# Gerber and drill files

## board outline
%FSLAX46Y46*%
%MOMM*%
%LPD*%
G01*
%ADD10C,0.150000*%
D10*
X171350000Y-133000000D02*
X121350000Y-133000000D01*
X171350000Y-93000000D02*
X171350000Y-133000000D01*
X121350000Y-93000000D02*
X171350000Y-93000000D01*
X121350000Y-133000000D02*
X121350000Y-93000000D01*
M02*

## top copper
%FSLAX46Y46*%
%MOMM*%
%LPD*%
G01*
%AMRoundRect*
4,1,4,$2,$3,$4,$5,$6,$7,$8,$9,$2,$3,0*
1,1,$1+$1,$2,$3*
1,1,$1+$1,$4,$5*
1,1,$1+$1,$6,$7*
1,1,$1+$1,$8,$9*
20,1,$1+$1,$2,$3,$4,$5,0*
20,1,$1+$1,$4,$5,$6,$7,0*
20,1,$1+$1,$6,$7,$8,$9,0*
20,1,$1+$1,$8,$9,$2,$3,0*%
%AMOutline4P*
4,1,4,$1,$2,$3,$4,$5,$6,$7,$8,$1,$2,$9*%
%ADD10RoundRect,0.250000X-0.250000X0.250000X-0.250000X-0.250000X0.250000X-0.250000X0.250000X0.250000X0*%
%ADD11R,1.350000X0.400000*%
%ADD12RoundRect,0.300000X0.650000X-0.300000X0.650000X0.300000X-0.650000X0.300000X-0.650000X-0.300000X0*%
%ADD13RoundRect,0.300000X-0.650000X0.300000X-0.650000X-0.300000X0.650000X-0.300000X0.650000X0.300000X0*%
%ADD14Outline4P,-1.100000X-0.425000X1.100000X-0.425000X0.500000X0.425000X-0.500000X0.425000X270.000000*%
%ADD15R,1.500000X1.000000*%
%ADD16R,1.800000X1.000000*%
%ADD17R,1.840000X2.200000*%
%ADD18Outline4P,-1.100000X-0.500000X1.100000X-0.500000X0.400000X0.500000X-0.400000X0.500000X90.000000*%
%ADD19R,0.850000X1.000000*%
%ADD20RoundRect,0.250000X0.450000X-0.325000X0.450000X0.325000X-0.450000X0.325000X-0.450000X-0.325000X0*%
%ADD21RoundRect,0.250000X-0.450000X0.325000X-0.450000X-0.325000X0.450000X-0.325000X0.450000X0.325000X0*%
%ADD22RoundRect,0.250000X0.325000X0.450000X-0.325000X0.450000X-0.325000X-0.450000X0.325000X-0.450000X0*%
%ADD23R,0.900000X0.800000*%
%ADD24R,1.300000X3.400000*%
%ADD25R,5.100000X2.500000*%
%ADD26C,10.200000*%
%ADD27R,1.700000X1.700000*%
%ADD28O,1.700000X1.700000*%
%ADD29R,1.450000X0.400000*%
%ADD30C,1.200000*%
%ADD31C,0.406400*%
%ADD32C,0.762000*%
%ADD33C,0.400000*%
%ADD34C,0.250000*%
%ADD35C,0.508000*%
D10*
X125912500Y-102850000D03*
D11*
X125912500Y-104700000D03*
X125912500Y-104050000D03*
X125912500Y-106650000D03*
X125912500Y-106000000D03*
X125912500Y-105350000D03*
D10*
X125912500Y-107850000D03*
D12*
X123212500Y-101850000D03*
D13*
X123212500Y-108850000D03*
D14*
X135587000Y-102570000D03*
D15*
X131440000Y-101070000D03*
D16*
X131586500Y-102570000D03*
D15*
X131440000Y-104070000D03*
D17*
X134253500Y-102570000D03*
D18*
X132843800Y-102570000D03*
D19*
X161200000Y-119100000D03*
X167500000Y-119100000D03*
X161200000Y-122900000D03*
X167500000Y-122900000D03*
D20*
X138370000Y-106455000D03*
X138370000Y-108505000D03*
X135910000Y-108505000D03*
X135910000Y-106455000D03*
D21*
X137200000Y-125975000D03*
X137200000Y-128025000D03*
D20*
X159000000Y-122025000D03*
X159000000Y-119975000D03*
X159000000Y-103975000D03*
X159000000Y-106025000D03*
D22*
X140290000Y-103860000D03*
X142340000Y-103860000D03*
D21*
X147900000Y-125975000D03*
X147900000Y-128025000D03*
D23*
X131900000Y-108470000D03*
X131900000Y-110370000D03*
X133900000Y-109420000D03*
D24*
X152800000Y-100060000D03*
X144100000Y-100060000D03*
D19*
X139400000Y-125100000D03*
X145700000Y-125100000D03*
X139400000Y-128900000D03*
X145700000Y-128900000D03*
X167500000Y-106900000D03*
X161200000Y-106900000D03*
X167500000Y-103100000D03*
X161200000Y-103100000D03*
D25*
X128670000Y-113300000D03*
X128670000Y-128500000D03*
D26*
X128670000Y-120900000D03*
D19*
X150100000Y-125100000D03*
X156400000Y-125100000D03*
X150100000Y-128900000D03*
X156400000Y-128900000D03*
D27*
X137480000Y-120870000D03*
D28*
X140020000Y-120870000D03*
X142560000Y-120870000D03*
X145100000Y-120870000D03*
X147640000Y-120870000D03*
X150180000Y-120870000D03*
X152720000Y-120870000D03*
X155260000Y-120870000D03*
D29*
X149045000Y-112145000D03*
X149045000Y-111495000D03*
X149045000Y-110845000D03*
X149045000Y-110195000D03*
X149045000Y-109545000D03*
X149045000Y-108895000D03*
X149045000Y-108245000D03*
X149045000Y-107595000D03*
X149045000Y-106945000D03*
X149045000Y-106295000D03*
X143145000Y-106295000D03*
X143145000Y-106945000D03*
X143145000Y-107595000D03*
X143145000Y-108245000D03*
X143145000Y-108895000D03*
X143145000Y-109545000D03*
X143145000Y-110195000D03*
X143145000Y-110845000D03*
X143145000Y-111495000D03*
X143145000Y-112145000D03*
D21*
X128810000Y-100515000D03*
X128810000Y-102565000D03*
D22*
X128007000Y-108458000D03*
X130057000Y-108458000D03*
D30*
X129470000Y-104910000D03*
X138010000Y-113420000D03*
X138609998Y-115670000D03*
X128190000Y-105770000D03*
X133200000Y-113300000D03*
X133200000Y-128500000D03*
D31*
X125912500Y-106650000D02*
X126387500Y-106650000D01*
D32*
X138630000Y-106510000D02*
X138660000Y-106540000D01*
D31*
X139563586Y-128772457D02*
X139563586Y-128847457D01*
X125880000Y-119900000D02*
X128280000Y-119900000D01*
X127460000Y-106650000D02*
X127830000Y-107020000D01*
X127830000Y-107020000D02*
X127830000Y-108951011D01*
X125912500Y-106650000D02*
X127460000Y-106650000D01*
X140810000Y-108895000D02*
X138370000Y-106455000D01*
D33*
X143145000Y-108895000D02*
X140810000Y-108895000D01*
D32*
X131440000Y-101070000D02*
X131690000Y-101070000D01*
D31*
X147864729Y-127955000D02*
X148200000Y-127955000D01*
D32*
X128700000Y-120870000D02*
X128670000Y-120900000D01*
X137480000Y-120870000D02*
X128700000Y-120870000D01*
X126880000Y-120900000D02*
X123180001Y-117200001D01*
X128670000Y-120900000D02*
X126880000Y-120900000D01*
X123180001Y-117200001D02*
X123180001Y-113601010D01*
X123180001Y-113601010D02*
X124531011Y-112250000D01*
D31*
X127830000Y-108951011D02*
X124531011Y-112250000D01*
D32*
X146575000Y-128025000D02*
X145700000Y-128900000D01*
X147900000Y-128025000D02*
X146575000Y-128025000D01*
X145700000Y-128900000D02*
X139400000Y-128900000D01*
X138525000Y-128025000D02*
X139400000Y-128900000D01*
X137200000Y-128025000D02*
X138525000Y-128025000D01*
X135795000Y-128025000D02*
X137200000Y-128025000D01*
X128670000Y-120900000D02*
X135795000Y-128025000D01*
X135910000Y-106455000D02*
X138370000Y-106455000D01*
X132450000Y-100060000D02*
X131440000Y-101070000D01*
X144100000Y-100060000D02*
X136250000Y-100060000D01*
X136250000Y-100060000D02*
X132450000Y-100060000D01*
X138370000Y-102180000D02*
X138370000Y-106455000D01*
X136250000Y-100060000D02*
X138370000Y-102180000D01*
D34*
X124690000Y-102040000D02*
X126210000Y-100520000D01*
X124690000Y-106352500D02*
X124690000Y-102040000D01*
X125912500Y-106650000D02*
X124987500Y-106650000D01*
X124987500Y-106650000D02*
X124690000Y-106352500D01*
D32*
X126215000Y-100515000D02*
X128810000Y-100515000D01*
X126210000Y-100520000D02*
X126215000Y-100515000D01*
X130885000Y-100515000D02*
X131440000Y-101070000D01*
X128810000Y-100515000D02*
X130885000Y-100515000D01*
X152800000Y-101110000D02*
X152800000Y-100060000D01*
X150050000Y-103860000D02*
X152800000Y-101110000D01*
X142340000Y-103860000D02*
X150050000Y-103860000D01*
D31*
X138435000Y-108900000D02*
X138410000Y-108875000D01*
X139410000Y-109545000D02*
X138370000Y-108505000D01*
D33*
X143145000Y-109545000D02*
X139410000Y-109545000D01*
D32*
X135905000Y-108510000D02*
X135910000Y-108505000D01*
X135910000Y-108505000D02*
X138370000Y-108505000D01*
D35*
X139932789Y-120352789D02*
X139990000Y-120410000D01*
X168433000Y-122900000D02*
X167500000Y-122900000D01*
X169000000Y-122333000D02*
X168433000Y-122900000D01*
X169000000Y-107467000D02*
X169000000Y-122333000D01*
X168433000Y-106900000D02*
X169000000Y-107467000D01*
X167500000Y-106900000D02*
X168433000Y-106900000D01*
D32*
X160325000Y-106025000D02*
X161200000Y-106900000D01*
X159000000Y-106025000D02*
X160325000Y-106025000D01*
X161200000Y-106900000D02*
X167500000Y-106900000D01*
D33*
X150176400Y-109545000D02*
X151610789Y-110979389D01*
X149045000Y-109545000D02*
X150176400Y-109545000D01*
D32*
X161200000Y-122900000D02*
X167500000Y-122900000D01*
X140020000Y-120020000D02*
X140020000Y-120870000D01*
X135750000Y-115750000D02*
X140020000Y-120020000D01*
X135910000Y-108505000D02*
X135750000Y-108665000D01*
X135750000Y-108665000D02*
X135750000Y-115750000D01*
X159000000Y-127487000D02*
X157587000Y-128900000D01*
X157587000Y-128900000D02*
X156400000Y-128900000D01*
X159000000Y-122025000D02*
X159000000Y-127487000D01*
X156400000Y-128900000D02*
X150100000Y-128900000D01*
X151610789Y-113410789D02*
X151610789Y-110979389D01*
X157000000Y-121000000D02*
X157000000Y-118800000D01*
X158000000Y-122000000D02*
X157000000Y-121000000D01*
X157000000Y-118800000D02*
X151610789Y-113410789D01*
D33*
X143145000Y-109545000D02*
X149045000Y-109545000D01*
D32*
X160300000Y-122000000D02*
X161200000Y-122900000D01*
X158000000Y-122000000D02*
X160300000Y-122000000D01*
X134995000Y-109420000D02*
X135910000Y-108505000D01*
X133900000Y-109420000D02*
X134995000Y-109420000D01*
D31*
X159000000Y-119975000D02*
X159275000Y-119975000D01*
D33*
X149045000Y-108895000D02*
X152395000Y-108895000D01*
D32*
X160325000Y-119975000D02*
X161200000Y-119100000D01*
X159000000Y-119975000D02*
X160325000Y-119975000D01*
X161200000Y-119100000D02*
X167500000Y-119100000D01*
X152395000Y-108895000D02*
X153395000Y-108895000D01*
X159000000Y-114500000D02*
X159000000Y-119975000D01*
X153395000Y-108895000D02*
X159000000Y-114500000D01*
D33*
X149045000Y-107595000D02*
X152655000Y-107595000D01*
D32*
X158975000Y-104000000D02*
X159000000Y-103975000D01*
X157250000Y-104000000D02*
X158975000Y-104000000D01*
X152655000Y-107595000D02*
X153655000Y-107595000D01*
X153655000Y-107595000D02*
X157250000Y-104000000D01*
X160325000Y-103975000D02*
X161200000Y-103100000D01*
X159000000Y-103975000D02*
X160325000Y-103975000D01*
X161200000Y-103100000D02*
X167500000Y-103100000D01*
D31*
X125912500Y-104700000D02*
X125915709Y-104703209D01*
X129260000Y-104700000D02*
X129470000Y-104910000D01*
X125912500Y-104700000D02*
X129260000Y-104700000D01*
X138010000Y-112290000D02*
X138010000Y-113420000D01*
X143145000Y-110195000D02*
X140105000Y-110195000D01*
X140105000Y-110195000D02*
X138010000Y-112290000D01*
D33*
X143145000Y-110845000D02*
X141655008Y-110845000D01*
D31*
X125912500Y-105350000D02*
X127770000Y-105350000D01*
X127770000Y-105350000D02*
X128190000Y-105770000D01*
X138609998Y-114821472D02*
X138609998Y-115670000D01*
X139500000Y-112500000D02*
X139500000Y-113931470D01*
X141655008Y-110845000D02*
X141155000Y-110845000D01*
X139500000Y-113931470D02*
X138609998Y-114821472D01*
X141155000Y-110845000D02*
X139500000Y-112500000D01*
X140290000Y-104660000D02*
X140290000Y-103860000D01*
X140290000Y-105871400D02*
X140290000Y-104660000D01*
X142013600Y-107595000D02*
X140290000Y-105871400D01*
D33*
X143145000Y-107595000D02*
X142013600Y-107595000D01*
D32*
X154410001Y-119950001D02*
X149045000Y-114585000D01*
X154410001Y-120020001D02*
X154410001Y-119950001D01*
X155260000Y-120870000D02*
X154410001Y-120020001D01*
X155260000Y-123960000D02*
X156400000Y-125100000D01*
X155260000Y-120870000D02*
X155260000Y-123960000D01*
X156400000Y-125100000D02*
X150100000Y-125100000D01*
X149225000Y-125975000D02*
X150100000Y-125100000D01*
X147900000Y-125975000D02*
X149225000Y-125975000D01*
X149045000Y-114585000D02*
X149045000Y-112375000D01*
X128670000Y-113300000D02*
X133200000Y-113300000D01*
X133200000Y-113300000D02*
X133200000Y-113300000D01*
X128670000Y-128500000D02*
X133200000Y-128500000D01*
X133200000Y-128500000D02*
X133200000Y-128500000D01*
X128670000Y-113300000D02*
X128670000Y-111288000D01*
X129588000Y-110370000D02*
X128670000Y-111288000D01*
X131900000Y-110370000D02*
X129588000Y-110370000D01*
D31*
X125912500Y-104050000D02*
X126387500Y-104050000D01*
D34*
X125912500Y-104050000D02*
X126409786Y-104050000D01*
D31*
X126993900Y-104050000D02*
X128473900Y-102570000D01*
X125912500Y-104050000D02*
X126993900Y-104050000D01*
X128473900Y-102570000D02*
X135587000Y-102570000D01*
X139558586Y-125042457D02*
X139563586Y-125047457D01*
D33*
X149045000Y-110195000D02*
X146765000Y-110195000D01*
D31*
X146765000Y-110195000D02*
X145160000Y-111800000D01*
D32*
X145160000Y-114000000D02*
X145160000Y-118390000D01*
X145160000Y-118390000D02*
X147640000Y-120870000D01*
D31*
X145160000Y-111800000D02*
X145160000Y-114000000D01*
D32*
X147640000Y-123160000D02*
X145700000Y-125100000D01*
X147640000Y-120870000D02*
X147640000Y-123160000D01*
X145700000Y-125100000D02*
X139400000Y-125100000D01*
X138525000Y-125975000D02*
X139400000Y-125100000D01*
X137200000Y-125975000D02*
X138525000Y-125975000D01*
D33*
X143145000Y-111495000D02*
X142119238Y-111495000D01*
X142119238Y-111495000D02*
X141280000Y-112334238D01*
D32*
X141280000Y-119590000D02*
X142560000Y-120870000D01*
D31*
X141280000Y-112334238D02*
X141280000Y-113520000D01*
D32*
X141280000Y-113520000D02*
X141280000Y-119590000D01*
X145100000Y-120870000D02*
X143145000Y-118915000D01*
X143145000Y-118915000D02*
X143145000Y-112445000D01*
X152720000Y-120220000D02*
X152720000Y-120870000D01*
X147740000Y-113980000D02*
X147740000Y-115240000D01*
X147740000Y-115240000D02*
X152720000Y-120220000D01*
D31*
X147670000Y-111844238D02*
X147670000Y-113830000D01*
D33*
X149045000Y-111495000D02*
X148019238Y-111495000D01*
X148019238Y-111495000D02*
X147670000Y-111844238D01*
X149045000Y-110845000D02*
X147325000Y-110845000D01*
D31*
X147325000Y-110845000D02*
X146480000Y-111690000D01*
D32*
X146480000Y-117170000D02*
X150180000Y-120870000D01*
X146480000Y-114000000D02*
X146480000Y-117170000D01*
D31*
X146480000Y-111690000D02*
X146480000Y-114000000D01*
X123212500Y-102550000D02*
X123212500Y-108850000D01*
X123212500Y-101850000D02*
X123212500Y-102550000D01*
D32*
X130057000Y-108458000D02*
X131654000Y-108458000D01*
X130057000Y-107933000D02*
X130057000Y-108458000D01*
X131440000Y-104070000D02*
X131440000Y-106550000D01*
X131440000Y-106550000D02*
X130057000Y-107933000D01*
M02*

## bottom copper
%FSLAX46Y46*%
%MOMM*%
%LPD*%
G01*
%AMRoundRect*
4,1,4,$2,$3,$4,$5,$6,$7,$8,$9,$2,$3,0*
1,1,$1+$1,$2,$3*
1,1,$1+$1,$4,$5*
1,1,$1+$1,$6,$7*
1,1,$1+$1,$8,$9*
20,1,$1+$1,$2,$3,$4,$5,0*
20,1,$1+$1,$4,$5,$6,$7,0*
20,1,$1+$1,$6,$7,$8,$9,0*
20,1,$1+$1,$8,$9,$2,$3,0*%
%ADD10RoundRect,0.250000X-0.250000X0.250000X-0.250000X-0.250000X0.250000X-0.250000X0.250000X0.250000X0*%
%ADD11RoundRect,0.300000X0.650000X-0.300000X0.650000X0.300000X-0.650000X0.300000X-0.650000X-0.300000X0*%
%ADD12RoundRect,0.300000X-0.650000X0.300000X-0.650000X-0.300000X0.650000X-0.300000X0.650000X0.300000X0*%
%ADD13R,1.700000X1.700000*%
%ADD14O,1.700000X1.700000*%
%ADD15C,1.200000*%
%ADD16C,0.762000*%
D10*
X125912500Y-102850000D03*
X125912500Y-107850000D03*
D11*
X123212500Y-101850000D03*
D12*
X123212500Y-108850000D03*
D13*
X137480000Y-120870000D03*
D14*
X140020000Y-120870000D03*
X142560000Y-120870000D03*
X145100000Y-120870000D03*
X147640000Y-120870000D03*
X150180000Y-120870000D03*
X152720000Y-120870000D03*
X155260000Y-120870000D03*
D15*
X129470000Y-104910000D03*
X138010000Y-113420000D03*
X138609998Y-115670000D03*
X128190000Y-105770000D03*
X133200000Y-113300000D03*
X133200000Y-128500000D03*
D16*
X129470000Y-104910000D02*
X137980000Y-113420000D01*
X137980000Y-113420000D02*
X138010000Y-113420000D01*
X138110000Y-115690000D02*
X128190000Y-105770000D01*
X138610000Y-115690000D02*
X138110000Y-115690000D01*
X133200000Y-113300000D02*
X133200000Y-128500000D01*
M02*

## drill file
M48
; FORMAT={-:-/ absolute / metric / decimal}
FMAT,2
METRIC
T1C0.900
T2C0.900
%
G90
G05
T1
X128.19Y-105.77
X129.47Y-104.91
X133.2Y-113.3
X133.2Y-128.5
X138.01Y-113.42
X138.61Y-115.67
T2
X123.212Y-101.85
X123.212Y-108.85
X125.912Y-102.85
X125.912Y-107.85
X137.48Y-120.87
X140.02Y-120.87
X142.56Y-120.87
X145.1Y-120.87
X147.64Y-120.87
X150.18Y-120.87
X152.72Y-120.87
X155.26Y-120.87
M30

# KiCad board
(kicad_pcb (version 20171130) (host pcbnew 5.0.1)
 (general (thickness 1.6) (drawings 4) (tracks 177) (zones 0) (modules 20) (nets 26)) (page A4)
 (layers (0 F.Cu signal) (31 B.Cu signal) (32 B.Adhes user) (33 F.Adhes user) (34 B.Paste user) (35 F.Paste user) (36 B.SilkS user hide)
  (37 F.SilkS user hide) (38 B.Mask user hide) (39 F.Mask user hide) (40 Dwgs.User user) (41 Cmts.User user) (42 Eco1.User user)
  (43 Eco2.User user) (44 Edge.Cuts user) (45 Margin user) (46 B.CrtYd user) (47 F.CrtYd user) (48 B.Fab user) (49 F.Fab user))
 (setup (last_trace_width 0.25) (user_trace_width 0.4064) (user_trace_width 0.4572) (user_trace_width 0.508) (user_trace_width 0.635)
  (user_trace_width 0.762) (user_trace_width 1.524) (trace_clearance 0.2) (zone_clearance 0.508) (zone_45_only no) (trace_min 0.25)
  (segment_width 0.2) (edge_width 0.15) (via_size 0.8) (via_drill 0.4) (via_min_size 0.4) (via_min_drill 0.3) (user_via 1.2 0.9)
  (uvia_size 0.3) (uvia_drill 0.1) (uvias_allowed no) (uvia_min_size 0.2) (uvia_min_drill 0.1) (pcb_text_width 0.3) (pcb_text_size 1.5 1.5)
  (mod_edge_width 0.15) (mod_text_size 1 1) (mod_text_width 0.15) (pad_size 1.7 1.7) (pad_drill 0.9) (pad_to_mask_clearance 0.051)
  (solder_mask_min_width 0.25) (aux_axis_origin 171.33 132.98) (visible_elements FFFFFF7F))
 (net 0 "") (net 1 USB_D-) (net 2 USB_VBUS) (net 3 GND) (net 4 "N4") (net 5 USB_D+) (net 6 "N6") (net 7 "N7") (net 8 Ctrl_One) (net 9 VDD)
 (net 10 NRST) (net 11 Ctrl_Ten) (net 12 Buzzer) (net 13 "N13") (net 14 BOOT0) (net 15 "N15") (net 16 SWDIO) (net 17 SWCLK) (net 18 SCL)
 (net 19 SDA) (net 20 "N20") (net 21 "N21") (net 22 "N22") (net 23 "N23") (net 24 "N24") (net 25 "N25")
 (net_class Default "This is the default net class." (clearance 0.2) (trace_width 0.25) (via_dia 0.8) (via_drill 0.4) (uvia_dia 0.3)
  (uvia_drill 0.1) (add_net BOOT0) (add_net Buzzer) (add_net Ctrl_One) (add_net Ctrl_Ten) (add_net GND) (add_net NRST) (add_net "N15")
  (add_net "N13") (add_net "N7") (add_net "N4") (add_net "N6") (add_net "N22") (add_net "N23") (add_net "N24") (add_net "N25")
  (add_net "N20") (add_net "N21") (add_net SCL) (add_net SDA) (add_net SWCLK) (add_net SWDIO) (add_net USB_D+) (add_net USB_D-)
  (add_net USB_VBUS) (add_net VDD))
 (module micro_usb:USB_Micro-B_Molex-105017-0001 (layer F.Cu) (at 124.45 105.35 270)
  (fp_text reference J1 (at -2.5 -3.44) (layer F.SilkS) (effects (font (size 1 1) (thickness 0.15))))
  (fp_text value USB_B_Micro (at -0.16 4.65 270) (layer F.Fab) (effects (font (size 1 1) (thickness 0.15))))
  (pad "" thru_hole roundrect (at -2.5 -1.4625 270) (size 1 1) (drill 0.9) (layers *.Cu *.Mask) (roundrect_rratio 0.25))
  (pad 2 smd rect (at -0.65 -1.4625 270) (size 0.4 1.35) (layers F.Cu F.Paste F.Mask) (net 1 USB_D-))
  (pad 1 smd rect (at -1.3 -1.4625 270) (size 0.4 1.35) (layers F.Cu F.Paste F.Mask) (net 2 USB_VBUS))
  (pad 5 smd rect (at 1.3 -1.4625 270) (size 0.4 1.35) (layers F.Cu F.Paste F.Mask) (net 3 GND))
  (pad 4 smd rect (at 0.65 -1.4625 270) (size 0.4 1.35) (layers F.Cu F.Paste F.Mask) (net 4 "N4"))
  (pad 3 smd rect (at 0 -1.4625 270) (size 0.4 1.35) (layers F.Cu F.Paste F.Mask) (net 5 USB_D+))
  (pad "" thru_hole roundrect (at 2.5 -1.4625 270) (size 1 1) (drill 0.9) (layers *.Cu *.Mask) (roundrect_rratio 0.25))
  (pad 6 thru_hole roundrect (at -3.5 1.2375 90) (size 1.2 1.9) (drill 0.9) (layers *.Cu *.Mask) (roundrect_rratio 0.25) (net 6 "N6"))
  (pad 6 thru_hole roundrect (at 3.5 1.2375 270) (size 1.2 1.9) (drill 0.9) (layers *.Cu *.Mask) (roundrect_rratio 0.25) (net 6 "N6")))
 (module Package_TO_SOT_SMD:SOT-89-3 (layer F.Cu) (at 132.92 102.57)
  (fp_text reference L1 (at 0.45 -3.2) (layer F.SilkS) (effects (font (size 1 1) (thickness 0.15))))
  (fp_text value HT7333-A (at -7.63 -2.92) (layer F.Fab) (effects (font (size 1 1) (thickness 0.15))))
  (pad 2 smd trapezoid (at 2.667 0 270) (size 1.6 0.85) (rect_delta 0 0.6) (layers F.Cu F.Paste F.Mask) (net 2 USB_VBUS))
  (pad 1 smd rect (at -1.48 -1.5 270) (size 1 1.5) (layers F.Cu F.Paste F.Mask) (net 3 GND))
  (pad 2 smd rect (at -1.3335 0 270) (size 1 1.8) (layers F.Cu F.Paste F.Mask) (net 2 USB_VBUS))
  (pad 3 smd rect (at -1.48 1.5 270) (size 1 1.5) (layers F.Cu F.Paste F.Mask) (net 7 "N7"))
  (pad 2 smd rect (at 1.3335 0 270) (size 2.2 1.84) (layers F.Cu F.Paste F.Mask) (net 2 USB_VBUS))
  (pad 2 smd trapezoid (at -0.0762 0 90) (size 1.5 1) (rect_delta 0 0.7) (layers F.Cu F.Paste F.Mask) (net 2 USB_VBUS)))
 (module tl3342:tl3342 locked (layer F.Cu) (at 164.35 121)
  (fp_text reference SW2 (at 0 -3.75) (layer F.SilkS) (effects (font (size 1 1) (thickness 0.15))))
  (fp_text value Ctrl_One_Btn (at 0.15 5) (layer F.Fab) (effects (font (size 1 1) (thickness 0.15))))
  (pad 1 smd rect (at -3.15 -1.9) (size 0.85 1) (layers F.Cu F.Paste F.Mask) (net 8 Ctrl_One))
  (pad 1 smd rect (at 3.15 -1.9) (size 0.85 1) (layers F.Cu F.Paste F.Mask) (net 8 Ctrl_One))
  (pad 2 smd rect (at -3.15 1.9) (size 0.85 1) (layers F.Cu F.Paste F.Mask) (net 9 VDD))
  (pad 2 smd rect (at 3.15 1.9) (size 0.85 1) (layers F.Cu F.Paste F.Mask) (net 9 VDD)))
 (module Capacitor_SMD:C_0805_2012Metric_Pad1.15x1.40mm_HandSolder (layer F.Cu) (at 138.37 107.48 90)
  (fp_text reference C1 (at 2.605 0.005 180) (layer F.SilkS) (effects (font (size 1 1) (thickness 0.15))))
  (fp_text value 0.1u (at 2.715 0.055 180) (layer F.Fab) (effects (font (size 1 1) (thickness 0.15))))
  (pad 2 smd roundrect (at 1.025 0 90) (size 1.15 1.4) (layers F.Cu F.Paste F.Mask) (roundrect_rratio 0.217391) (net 3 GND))
  (pad 1 smd roundrect (at -1.025 0 90) (size 1.15 1.4) (layers F.Cu F.Paste F.Mask) (roundrect_rratio 0.217391) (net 9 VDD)))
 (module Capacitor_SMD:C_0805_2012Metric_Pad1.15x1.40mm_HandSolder (layer F.Cu) (at 135.91 107.48 90)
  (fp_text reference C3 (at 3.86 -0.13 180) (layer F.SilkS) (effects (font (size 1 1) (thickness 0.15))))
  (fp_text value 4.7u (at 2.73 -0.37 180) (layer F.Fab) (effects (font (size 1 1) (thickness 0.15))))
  (pad 1 smd roundrect (at -1.025 0 90) (size 1.15 1.4) (layers F.Cu F.Paste F.Mask) (roundrect_rratio 0.217391) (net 9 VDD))
  (pad 2 smd roundrect (at 1.025 0 90) (size 1.15 1.4) (layers F.Cu F.Paste F.Mask) (roundrect_rratio 0.217391) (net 3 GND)))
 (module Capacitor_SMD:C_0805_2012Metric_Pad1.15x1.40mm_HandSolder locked (layer F.Cu) (at 137.2 127 270)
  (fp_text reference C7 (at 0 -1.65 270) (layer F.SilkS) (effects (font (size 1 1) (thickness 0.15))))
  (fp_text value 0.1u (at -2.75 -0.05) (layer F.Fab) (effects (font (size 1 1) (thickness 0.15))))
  (pad 1 smd roundrect (at -1.025 0 270) (size 1.15 1.4) (layers F.Cu F.Paste F.Mask) (roundrect_rratio 0.217391) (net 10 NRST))
  (pad 2 smd roundrect (at 1.025 0 270) (size 1.15 1.4) (layers F.Cu F.Paste F.Mask) (roundrect_rratio 0.217391) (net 3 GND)))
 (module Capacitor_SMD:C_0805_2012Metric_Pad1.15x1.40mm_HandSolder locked (layer F.Cu) (at 159 121 90)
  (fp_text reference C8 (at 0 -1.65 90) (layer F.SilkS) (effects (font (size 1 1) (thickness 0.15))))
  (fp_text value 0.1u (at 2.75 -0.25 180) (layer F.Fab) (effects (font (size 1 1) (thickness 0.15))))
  (pad 1 smd roundrect (at -1.025 0 90) (size 1.15 1.4) (layers F.Cu F.Paste F.Mask) (roundrect_rratio 0.217391) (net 9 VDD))
  (pad 2 smd roundrect (at 1.025 0 90) (size 1.15 1.4) (layers F.Cu F.Paste F.Mask) (roundrect_rratio 0.217391) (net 8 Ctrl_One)))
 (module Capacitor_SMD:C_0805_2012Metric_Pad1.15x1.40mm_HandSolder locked (layer F.Cu) (at 159 105 90)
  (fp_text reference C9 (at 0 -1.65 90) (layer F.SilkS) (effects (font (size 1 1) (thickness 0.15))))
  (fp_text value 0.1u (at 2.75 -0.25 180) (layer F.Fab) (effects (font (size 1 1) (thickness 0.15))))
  (pad 2 smd roundrect (at 1.025 0 90) (size 1.15 1.4) (layers F.Cu F.Paste F.Mask) (roundrect_rratio 0.217391) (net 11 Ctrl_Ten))
  (pad 1 smd roundrect (at -1.025 0 90) (size 1.15 1.4) (layers F.Cu F.Paste F.Mask) (roundrect_rratio 0.217391) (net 9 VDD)))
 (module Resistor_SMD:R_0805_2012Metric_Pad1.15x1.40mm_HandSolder (layer F.Cu) (at 141.315 103.86 180)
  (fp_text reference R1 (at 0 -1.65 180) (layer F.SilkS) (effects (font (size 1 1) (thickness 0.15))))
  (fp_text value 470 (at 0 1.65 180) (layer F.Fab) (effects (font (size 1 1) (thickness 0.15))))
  (pad 2 smd roundrect (at 1.025 0 180) (size 1.15 1.4) (layers F.Cu F.Paste F.Mask) (roundrect_rratio 0.217391) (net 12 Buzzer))
  (pad 1 smd roundrect (at -1.025 0 180) (size 1.15 1.4) (layers F.Cu F.Paste F.Mask) (roundrect_rratio 0.217391) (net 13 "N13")))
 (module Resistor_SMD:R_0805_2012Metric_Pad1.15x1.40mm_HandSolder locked (layer F.Cu) (at 147.9 127 270)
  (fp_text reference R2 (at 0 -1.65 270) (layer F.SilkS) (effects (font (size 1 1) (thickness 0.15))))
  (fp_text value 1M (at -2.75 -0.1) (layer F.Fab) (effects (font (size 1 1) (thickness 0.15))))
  (pad 1 smd roundrect (at -1.025 0 270) (size 1.15 1.4) (layers F.Cu F.Paste F.Mask) (roundrect_rratio 0.217391) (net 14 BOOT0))
  (pad 2 smd roundrect (at 1.025 0 270) (size 1.15 1.4) (layers F.Cu F.Paste F.Mask) (roundrect_rratio 0.217391) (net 3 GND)))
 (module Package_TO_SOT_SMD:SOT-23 (layer F.Cu) (at 132.9 109.42)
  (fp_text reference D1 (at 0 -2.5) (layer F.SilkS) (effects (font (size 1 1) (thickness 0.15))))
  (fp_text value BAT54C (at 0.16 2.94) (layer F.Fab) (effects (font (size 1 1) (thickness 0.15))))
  (pad 1 smd rect (at -1 -0.95) (size 0.9 0.8) (layers F.Cu F.Paste F.Mask) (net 7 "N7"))
  (pad 2 smd rect (at -1 0.95) (size 0.9 0.8) (layers F.Cu F.Paste F.Mask) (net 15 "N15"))
  (pad 3 smd rect (at 1 0) (size 0.9 0.8) (layers F.Cu F.Paste F.Mask) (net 9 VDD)))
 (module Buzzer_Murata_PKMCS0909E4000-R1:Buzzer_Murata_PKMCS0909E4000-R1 (layer F.Cu) (at 148.45 100.06 180)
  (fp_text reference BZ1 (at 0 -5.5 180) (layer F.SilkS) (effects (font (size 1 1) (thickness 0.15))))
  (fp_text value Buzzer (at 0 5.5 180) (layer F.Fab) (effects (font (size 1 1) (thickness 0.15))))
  (pad 1 smd rect (at -4.35 0 180) (size 1.3 3.4) (layers F.Cu F.Paste F.Mask) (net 13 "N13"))
  (pad 2 smd rect (at 4.35 0 180) (size 1.3 3.4) (layers F.Cu F.Paste F.Mask) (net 3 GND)))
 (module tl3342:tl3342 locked (layer F.Cu) (at 142.55 127)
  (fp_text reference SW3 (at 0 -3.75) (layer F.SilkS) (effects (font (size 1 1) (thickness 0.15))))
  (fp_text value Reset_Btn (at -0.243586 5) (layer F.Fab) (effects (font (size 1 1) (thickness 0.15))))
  (pad 1 smd rect (at -3.15 -1.9) (size 0.85 1) (layers F.Cu F.Paste F.Mask) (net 10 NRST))
  (pad 1 smd rect (at 3.15 -1.9) (size 0.85 1) (layers F.Cu F.Paste F.Mask) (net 10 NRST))
  (pad 2 smd rect (at -3.15 1.9) (size 0.85 1) (layers F.Cu F.Paste F.Mask) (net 3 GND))
  (pad 2 smd rect (at 3.15 1.9) (size 0.85 1) (layers F.Cu F.Paste F.Mask) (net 3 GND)))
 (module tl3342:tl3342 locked (layer F.Cu) (at 164.35 105)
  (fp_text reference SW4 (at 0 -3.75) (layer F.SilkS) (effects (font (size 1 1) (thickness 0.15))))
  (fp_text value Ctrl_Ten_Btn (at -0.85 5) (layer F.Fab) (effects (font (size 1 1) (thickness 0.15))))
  (pad 2 smd rect (at 3.15 1.9) (size 0.85 1) (layers F.Cu F.Paste F.Mask) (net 9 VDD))
  (pad 2 smd rect (at -3.15 1.9) (size 0.85 1) (layers F.Cu F.Paste F.Mask) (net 9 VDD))
  (pad 1 smd rect (at 3.15 -1.9) (size 0.85 1) (layers F.Cu F.Paste F.Mask) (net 11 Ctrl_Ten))
  (pad 1 smd rect (at -3.15 -1.9) (size 0.85 1) (layers F.Cu F.Paste F.Mask) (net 11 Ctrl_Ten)))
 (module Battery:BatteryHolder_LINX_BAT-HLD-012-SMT (layer F.Cu) (at 128.67 120.9 270)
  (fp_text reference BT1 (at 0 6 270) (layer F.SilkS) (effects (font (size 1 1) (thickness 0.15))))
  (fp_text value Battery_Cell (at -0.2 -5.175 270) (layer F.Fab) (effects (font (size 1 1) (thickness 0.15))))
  (pad 1 smd rect (at -7.6 0 270) (size 2.5 5.1) (layers F.Cu F.Paste F.Mask) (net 15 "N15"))
  (pad 1 smd rect (at 7.6 0 270) (size 2.5 5.1) (layers F.Cu F.Paste F.Mask) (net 15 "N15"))
  (pad 2 smd circle (at 0 0 270) (size 10.2 10.2) (layers F.Cu F.Paste F.Mask) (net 3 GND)))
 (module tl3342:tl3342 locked (layer F.Cu) (at 153.25 127)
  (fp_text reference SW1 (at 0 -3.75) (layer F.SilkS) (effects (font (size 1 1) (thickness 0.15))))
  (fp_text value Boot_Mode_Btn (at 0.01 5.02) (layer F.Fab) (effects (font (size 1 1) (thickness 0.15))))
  (pad 1 smd rect (at -3.15 -1.9) (size 0.85 1) (layers F.Cu F.Paste F.Mask) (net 14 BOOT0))
  (pad 1 smd rect (at 3.15 -1.9) (size 0.85 1) (layers F.Cu F.Paste F.Mask) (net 14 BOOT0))
  (pad 2 smd rect (at -3.15 1.9) (size 0.85 1) (layers F.Cu F.Paste F.Mask) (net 9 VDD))
  (pad 2 smd rect (at 3.15 1.9) (size 0.85 1) (layers F.Cu F.Paste F.Mask) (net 9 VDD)))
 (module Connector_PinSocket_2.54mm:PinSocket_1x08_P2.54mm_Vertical (layer F.Cu) (at 137.48 120.87 90)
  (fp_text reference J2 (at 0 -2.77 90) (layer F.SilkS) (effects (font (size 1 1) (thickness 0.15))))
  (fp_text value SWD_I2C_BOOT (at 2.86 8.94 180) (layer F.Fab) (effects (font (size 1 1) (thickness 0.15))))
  (pad 1 thru_hole rect (at 0 0 90) (size 1.7 1.7) (drill 0.9) (layers *.Cu *.Mask) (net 3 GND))
  (pad 2 thru_hole oval (at 0 2.54 90) (size 1.7 1.7) (drill 0.9) (layers *.Cu *.Mask) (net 9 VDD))
  (pad 3 thru_hole oval (at 0 5.08 90) (size 1.7 1.7) (drill 0.9) (layers *.Cu *.Mask) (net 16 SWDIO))
  (pad 4 thru_hole oval (at 0 7.62 90) (size 1.7 1.7) (drill 0.9) (layers *.Cu *.Mask) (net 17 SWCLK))
  (pad 5 thru_hole oval (at 0 10.16 90) (size 1.7 1.7) (drill 0.9) (layers *.Cu *.Mask) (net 10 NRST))
  (pad 6 thru_hole oval (at 0 12.7 90) (size 1.7 1.7) (drill 0.9) (layers *.Cu *.Mask) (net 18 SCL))
  (pad 7 thru_hole oval (at 0 15.24 90) (size 1.7 1.7) (drill 0.9) (layers *.Cu *.Mask) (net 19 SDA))
  (pad 8 thru_hole oval (at 0 17.78 90) (size 1.7 1.7) (drill 0.9) (layers *.Cu *.Mask) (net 14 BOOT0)))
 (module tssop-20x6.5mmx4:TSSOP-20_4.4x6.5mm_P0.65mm (layer F.Cu) (at 146.095 109.22 180)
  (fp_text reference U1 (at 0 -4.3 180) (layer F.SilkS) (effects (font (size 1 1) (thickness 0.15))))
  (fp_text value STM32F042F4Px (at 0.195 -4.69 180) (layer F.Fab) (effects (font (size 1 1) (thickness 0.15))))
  (pad 1 smd rect (at -2.95 -2.925 180) (size 1.45 0.4) (layers F.Cu F.Paste F.Mask) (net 14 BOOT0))
  (pad 2 smd rect (at -2.95 -2.275 180) (size 1.45 0.4) (layers F.Cu F.Paste F.Mask) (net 19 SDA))
  (pad 3 smd rect (at -2.95 -1.625 180) (size 1.45 0.4) (layers F.Cu F.Paste F.Mask) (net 18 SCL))
  (pad 4 smd rect (at -2.95 -0.975 180) (size 1.45 0.4) (layers F.Cu F.Paste F.Mask) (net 10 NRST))
  (pad 5 smd rect (at -2.95 -0.325 180) (size 1.45 0.4) (layers F.Cu F.Paste F.Mask) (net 9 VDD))
  (pad 6 smd rect (at -2.95 0.325 180) (size 1.45 0.4) (layers F.Cu F.Paste F.Mask) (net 8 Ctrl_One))
  (pad 7 smd rect (at -2.95 0.975 180) (size 1.45 0.4) (layers F.Cu F.Paste F.Mask) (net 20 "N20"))
  (pad 8 smd rect (at -2.95 1.625 180) (size 1.45 0.4) (layers F.Cu F.Paste F.Mask) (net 11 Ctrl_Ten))
  (pad 9 smd rect (at -2.95 2.275 180) (size 1.45 0.4) (layers F.Cu F.Paste F.Mask) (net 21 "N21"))
  (pad 10 smd rect (at -2.95 2.925 180) (size 1.45 0.4) (layers F.Cu F.Paste F.Mask) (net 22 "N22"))
  (pad 11 smd rect (at 2.95 2.925 180) (size 1.45 0.4) (layers F.Cu F.Paste F.Mask) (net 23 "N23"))
  (pad 12 smd rect (at 2.95 2.275 180) (size 1.45 0.4) (layers F.Cu F.Paste F.Mask) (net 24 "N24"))
  (pad 13 smd rect (at 2.95 1.625 180) (size 1.45 0.4) (layers F.Cu F.Paste F.Mask) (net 12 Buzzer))
  (pad 14 smd rect (at 2.95 0.975 180) (size 1.45 0.4) (layers F.Cu F.Paste F.Mask) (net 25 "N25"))
  (pad 15 smd rect (at 2.95 0.325 180) (size 1.45 0.4) (layers F.Cu F.Paste F.Mask) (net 3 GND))
  (pad 16 smd rect (at 2.95 -0.325 180) (size 1.45 0.4) (layers F.Cu F.Paste F.Mask) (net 9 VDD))
  (pad 17 smd rect (at 2.95 -0.975 180) (size 1.45 0.4) (layers F.Cu F.Paste F.Mask) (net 1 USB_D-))
  (pad 18 smd rect (at 2.95 -1.625 180) (size 1.45 0.4) (layers F.Cu F.Paste F.Mask) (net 5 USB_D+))
  (pad 19 smd rect (at 2.95 -2.275 180) (size 1.45 0.4) (layers F.Cu F.Paste F.Mask) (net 16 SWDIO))
  (pad 20 smd rect (at 2.95 -2.925 180) (size 1.45 0.4) (layers F.Cu F.Paste F.Mask) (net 17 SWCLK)))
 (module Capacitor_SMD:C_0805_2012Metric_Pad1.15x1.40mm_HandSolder (layer F.Cu) (at 128.81 101.54 270)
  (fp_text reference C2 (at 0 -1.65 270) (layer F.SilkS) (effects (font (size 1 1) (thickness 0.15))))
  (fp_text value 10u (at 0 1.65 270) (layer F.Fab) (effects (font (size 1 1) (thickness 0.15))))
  (pad 1 smd roundrect (at -1.025 0 270) (size 1.15 1.4) (layers F.Cu F.Paste F.Mask) (roundrect_rratio 0.217391) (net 3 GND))
  (pad 2 smd roundrect (at 1.025 0 270) (size 1.15 1.4) (layers F.Cu F.Paste F.Mask) (roundrect_rratio 0.217391) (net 2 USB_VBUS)))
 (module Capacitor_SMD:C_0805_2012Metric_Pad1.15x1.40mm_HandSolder (layer F.Cu) (at 129.032 108.458 180)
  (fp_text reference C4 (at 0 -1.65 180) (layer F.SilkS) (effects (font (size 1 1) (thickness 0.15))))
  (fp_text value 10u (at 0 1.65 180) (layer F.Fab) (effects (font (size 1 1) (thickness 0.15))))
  (pad 2 smd roundrect (at 1.025 0 180) (size 1.15 1.4) (layers F.Cu F.Paste F.Mask) (roundrect_rratio 0.217391) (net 3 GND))
  (pad 1 smd roundrect (at -1.025 0 180) (size 1.15 1.4) (layers F.Cu F.Paste F.Mask) (roundrect_rratio 0.217391) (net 7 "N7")))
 (gr_line (start 171.35 133) (end 121.35 133) (layer Edge.Cuts) (width 0.15))
 (gr_line (start 171.35 93) (end 171.35 133) (layer Edge.Cuts) (width 0.15))
 (gr_line (start 121.35 93) (end 171.35 93) (layer Edge.Cuts) (width 0.15))
 (gr_line (start 121.35 133) (end 121.35 93) (layer Edge.Cuts) (width 0.15))
 (segment (start 125.9125 106.65) (end 126.3875 106.65) (width 0.4064) (layer F.Cu) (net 3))
 (segment (start 138.63 106.51) (end 138.66 106.54) (width 0.762) (layer F.Cu) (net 3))
 (segment (start 139.563586 128.772457) (end 139.563586 128.847457) (width 0.4064) (layer F.Cu) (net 3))
 (segment (start 125.88 119.9) (end 128.28 119.9) (width 0.4064) (layer F.Cu) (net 3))
 (segment (start 127.46 106.65) (end 127.83 107.02) (width 0.4064) (layer F.Cu) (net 3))
 (segment (start 127.83 107.02) (end 127.83 108.951011) (width 0.4064) (layer F.Cu) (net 3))
 (segment (start 125.9125 106.65) (end 127.46 106.65) (width 0.4064) (layer F.Cu) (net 3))
 (segment (start 140.81 108.895) (end 138.37 106.455) (width 0.4064) (layer F.Cu) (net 3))
 (segment (start 143.145 108.895) (end 140.81 108.895) (width 0.4) (layer F.Cu) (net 3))
 (segment (start 131.44 101.07) (end 131.69 101.07) (width 0.762) (layer F.Cu) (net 3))
 (segment (start 147.864729 127.955) (end 148.2 127.955) (width 0.4064) (layer F.Cu) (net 3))
 (segment (start 128.7 120.87) (end 128.67 120.9) (width 0.762) (layer F.Cu) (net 3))
 (segment (start 137.48 120.87) (end 128.7 120.87) (width 0.762) (layer F.Cu) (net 3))
 (segment (start 126.88 120.9) (end 123.180001 117.200001) (width 0.762) (layer F.Cu) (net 3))
 (segment (start 128.67 120.9) (end 126.88 120.9) (width 0.762) (layer F.Cu) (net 3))
 (segment (start 123.180001 117.200001) (end 123.180001 113.60101) (width 0.762) (layer F.Cu) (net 3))
 (segment (start 123.180001 113.60101) (end 124.531011 112.25) (width 0.762) (layer F.Cu) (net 3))
 (segment (start 127.83 108.951011) (end 124.531011 112.25) (width 0.4064) (layer F.Cu) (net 3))
 (segment (start 146.575 128.025) (end 145.7 128.9) (width 0.762) (layer F.Cu) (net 3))
 (segment (start 147.9 128.025) (end 146.575 128.025) (width 0.762) (layer F.Cu) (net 3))
 (segment (start 145.7 128.9) (end 139.4 128.9) (width 0.762) (layer F.Cu) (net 3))
 (segment (start 138.525 128.025) (end 139.4 128.9) (width 0.762) (layer F.Cu) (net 3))
 (segment (start 137.2 128.025) (end 138.525 128.025) (width 0.762) (layer F.Cu) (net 3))
 (segment (start 135.795 128.025) (end 137.2 128.025) (width 0.762) (layer F.Cu) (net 3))
 (segment (start 128.67 120.9) (end 135.795 128.025) (width 0.762) (layer F.Cu) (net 3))
 (segment (start 135.91 106.455) (end 138.37 106.455) (width 0.762) (layer F.Cu) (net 3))
 (segment (start 132.45 100.06) (end 131.44 101.07) (width 0.762) (layer F.Cu) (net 3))
 (segment (start 144.1 100.06) (end 136.25 100.06) (width 0.762) (layer F.Cu) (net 3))
 (segment (start 136.25 100.06) (end 132.45 100.06) (width 0.762) (layer F.Cu) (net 3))
 (segment (start 138.37 102.18) (end 138.37 106.455) (width 0.762) (layer F.Cu) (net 3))
 (segment (start 136.25 100.06) (end 138.37 102.18) (width 0.762) (layer F.Cu) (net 3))
 (segment (start 124.69 102.04) (end 126.21 100.52) (width 0.25) (layer F.Cu) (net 3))
 (segment (start 124.69 106.3525) (end 124.69 102.04) (width 0.25) (layer F.Cu) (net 3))
 (segment (start 125.9125 106.65) (end 124.9875 106.65) (width 0.25) (layer F.Cu) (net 3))
 (segment (start 124.9875 106.65) (end 124.69 106.3525) (width 0.25) (layer F.Cu) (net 3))
 (segment (start 126.215 100.515) (end 128.81 100.515) (width 0.762) (layer F.Cu) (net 3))
 (segment (start 126.21 100.52) (end 126.215 100.515) (width 0.762) (layer F.Cu) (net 3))
 (segment (start 130.885 100.515) (end 131.44 101.07) (width 0.762) (layer F.Cu) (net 3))
 (segment (start 128.81 100.515) (end 130.885 100.515) (width 0.762) (layer F.Cu) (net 3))
 (segment (start 152.8 101.11) (end 152.8 100.06) (width 0.762) (layer F.Cu) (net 13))
 (segment (start 150.05 103.86) (end 152.8 101.11) (width 0.762) (layer F.Cu) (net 13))
 (segment (start 142.34 103.86) (end 150.05 103.86) (width 0.762) (layer F.Cu) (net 13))
 (segment (start 138.435 108.9) (end 138.41 108.875) (width 0.4064) (layer F.Cu) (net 9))
 (segment (start 139.41 109.545) (end 138.37 108.505) (width 0.4064) (layer F.Cu) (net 9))
 (segment (start 143.145 109.545) (end 139.41 109.545) (width 0.4) (layer F.Cu) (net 9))
 (segment (start 135.905 108.51) (end 135.91 108.505) (width 0.762) (layer F.Cu) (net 9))
 (segment (start 135.91 108.505) (end 138.37 108.505) (width 0.762) (layer F.Cu) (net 9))
 (segment (start 139.932789 120.352789) (end 139.99 120.41) (width 0.508) (layer F.Cu) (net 9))
 (segment (start 168.433 122.9) (end 167.5 122.9) (width 0.508) (layer F.Cu) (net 9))
 (segment (start 169 122.333) (end 168.433 122.9) (width 0.508) (layer F.Cu) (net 9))
 (segment (start 169 107.467) (end 169 122.333) (width 0.508) (layer F.Cu) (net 9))
 (segment (start 168.433 106.9) (end 169 107.467) (width 0.508) (layer F.Cu) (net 9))
 (segment (start 167.5 106.9) (end 168.433 106.9) (width 0.508) (layer F.Cu) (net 9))
 (segment (start 160.325 106.025) (end 161.2 106.9) (width 0.762) (layer F.Cu) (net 9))
 (segment (start 159 106.025) (end 160.325 106.025) (width 0.762) (layer F.Cu) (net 9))
 (segment (start 161.2 106.9) (end 167.5 106.9) (width 0.762) (layer F.Cu) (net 9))
 (segment (start 150.1764 109.545) (end 151.610789 110.979389) (width 0.4) (layer F.Cu) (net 9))
 (segment (start 149.045 109.545) (end 150.1764 109.545) (width 0.4) (layer F.Cu) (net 9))
 (segment (start 161.2 122.9) (end 167.5 122.9) (width 0.762) (layer F.Cu) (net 9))
 (segment (start 140.02 120.02) (end 140.02 120.87) (width 0.762) (layer F.Cu) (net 9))
 (segment (start 135.75 115.75) (end 140.02 120.02) (width 0.762) (layer F.Cu) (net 9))
 (segment (start 135.91 108.505) (end 135.75 108.665) (width 0.762) (layer F.Cu) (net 9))
 (segment (start 135.75 108.665) (end 135.75 115.75) (width 0.762) (layer F.Cu) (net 9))
 (segment (start 159 127.487) (end 157.587 128.9) (width 0.762) (layer F.Cu) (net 9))
 (segment (start 157.587 128.9) (end 156.4 128.9) (width 0.762) (layer F.Cu) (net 9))
 (segment (start 159 122.025) (end 159 127.487) (width 0.762) (layer F.Cu) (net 9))
 (segment (start 156.4 128.9) (end 150.1 128.9) (width 0.762) (layer F.Cu) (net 9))
 (segment (start 151.610789 113.410789) (end 151.610789 110.979389) (width 0.762) (layer F.Cu) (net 9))
 (segment (start 157 121) (end 157 118.8) (width 0.762) (layer F.Cu) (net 9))
 (segment (start 158 122) (end 157 121) (width 0.762) (layer F.Cu) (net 9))
 (segment (start 157 118.8) (end 151.610789 113.410789) (width 0.762) (layer F.Cu) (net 9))
 (segment (start 143.145 109.545) (end 149.045 109.545) (width 0.4) (layer F.Cu) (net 9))
 (segment (start 160.3 122) (end 161.2 122.9) (width 0.762) (layer F.Cu) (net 9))
 (segment (start 158 122) (end 160.3 122) (width 0.762) (layer F.Cu) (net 9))
 (segment (start 134.995 109.42) (end 135.91 108.505) (width 0.762) (layer F.Cu) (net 9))
 (segment (start 133.9 109.42) (end 134.995 109.42) (width 0.762) (layer F.Cu) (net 9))
 (segment (start 159 119.975) (end 159.275 119.975) (width 0.4064) (layer F.Cu) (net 8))
 (segment (start 149.045 108.895) (end 152.395 108.895) (width 0.4) (layer F.Cu) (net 8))
 (segment (start 160.325 119.975) (end 161.2 119.1) (width 0.762) (layer F.Cu) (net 8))
 (segment (start 159 119.975) (end 160.325 119.975) (width 0.762) (layer F.Cu) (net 8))
 (segment (start 161.2 119.1) (end 167.5 119.1) (width 0.762) (layer F.Cu) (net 8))
 (segment (start 152.395 108.895) (end 153.395 108.895) (width 0.762) (layer F.Cu) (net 8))
 (segment (start 159 114.5) (end 159 119.975) (width 0.762) (layer F.Cu) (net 8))
 (segment (start 153.395 108.895) (end 159 114.5) (width 0.762) (layer F.Cu) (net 8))
 (segment (start 149.045 107.595) (end 152.655 107.595) (width 0.4) (layer F.Cu) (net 11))
 (segment (start 158.975 104) (end 159 103.975) (width 0.762) (layer F.Cu) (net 11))
 (segment (start 157.25 104) (end 158.975 104) (width 0.762) (layer F.Cu) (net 11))
 (segment (start 152.655 107.595) (end 153.655 107.595) (width 0.762) (layer F.Cu) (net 11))
 (segment (start 153.655 107.595) (end 157.25 104) (width 0.762) (layer F.Cu) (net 11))
 (segment (start 160.325 103.975) (end 161.2 103.1) (width 0.762) (layer F.Cu) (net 11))
 (segment (start 159 103.975) (end 160.325 103.975) (width 0.762) (layer F.Cu) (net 11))
 (segment (start 161.2 103.1) (end 167.5 103.1) (width 0.762) (layer F.Cu) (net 11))
 (segment (start 125.9125 104.7) (end 125.915709 104.703209) (width 0.4064) (layer F.Cu) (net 1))
 (via (at 129.47 104.91) (size 1.2) (drill 0.9) (layers F.Cu B.Cu) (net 1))
 (segment (start 129.26 104.7) (end 129.47 104.91) (width 0.4064) (layer F.Cu) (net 1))
 (segment (start 125.9125 104.7) (end 129.26 104.7) (width 0.4064) (layer F.Cu) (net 1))
 (via (at 138.01 113.42) (size 1.2) (drill 0.9) (layers F.Cu B.Cu) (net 1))
 (segment (start 129.47 104.91) (end 137.98 113.42) (width 0.762) (layer B.Cu) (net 1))
 (segment (start 137.98 113.42) (end 138.01 113.42) (width 0.762) (layer B.Cu) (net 1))
 (segment (start 138.01 112.29) (end 138.01 113.42) (width 0.4064) (layer F.Cu) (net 1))
 (segment (start 143.145 110.195) (end 140.105 110.195) (width 0.4064) (layer F.Cu) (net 1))
 (segment (start 140.105 110.195) (end 138.01 112.29) (width 0.4064) (layer F.Cu) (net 1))
 (segment (start 143.145 110.845) (end 141.655008 110.845) (width 0.4) (layer F.Cu) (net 5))
 (via (at 138.609998 115.67) (size 1.2) (drill 0.9) (layers F.Cu B.Cu) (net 5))
 (via (at 128.19 105.77) (size 1.2) (drill 0.9) (layers F.Cu B.Cu) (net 5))
 (segment (start 125.9125 105.35) (end 127.77 105.35) (width 0.4064) (layer F.Cu) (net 5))
 (segment (start 127.77 105.35) (end 128.19 105.77) (width 0.4064) (layer F.Cu) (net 5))
 (segment (start 138.11 115.69) (end 128.19 105.77) (width 0.762) (layer B.Cu) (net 5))
 (segment (start 138.61 115.69) (end 138.11 115.69) (width 0.762) (layer B.Cu) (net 5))
 (segment (start 138.609998 114.821472) (end 138.609998 115.67) (width 0.4064) (layer F.Cu) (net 5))
 (segment (start 139.5 112.5) (end 139.5 113.93147) (width 0.4064) (layer F.Cu) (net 5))
 (segment (start 141.655008 110.845) (end 141.155 110.845) (width 0.4064) (layer F.Cu) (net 5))
 (segment (start 139.5 113.93147) (end 138.609998 114.821472) (width 0.4064) (layer F.Cu) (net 5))
 (segment (start 141.155 110.845) (end 139.5 112.5) (width 0.4064) (layer F.Cu) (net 5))
 (segment (start 140.29 104.66) (end 140.29 103.86) (width 0.4064) (layer F.Cu) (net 12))
 (segment (start 140.29 105.8714) (end 140.29 104.66) (width 0.4064) (layer F.Cu) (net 12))
 (segment (start 142.0136 107.595) (end 140.29 105.8714) (width 0.4064) (layer F.Cu) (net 12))
 (segment (start 143.145 107.595) (end 142.0136 107.595) (width 0.4) (layer F.Cu) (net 12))
 (segment (start 154.410001 119.950001) (end 149.045 114.585) (width 0.762) (layer F.Cu) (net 14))
 (segment (start 154.410001 120.020001) (end 154.410001 119.950001) (width 0.762) (layer F.Cu) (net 14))
 (segment (start 155.26 120.87) (end 154.410001 120.020001) (width 0.762) (layer F.Cu) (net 14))
 (segment (start 155.26 123.96) (end 156.4 125.1) (width 0.762) (layer F.Cu) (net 14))
 (segment (start 155.26 120.87) (end 155.26 123.96) (width 0.762) (layer F.Cu) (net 14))
 (segment (start 156.4 125.1) (end 150.1 125.1) (width 0.762) (layer F.Cu) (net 14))
 (segment (start 149.225 125.975) (end 150.1 125.1) (width 0.762) (layer F.Cu) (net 14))
 (segment (start 147.9 125.975) (end 149.225 125.975) (width 0.762) (layer F.Cu) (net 14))
 (segment (start 149.045 114.585) (end 149.045 112.375) (width 0.762) (layer F.Cu) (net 14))
 (segment (start 128.67 113.3) (end 133.2 113.3) (width 0.762) (layer F.Cu) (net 15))
 (segment (start 133.2 113.3) (end 133.2 113.3) (width 0.762) (layer F.Cu) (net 15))
 (via (at 133.2 113.3) (size 1.2) (drill 0.9) (layers F.Cu B.Cu) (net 15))
 (segment (start 128.67 128.5) (end 133.2 128.5) (width 0.762) (layer F.Cu) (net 15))
 (segment (start 133.2 128.5) (end 133.2 128.5) (width 0.762) (layer F.Cu) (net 15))
 (via (at 133.2 128.5) (size 1.2) (drill 0.9) (layers F.Cu B.Cu) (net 15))
 (segment (start 133.2 113.3) (end 133.2 128.5) (width 0.762) (layer B.Cu) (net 15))
 (segment (start 128.67 113.3) (end 128.67 111.288) (width 0.762) (layer F.Cu) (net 15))
 (segment (start 129.588 110.37) (end 128.67 111.288) (width 0.762) (layer F.Cu) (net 15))
 (segment (start 131.9 110.37) (end 129.588 110.37) (width 0.762) (layer F.Cu) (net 15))
 (segment (start 125.9125 104.05) (end 126.3875 104.05) (width 0.4064) (layer F.Cu) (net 2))
 (segment (start 125.9125 104.05) (end 126.409786 104.05) (width 0.25) (layer F.Cu) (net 2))
 (segment (start 126.9939 104.05) (end 128.4739 102.57) (width 0.4064) (layer F.Cu) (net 2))
 (segment (start 125.9125 104.05) (end 126.9939 104.05) (width 0.4064) (layer F.Cu) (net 2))
 (segment (start 128.4739 102.57) (end 135.587 102.57) (width 0.4064) (layer F.Cu) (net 2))
 (segment (start 139.558586 125.042457) (end 139.563586 125.047457) (width 0.4064) (layer F.Cu) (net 10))
 (segment (start 149.045 110.195) (end 146.765 110.195) (width 0.4) (layer F.Cu) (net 10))
 (segment (start 146.765 110.195) (end 145.16 111.8) (width 0.4064) (layer F.Cu) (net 10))
 (segment (start 145.16 114) (end 145.16 118.39) (width 0.762) (layer F.Cu) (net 10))
 (segment (start 145.16 118.39) (end 147.64 120.87) (width 0.762) (layer F.Cu) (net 10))
 (segment (start 145.16 111.8) (end 145.16 114) (width 0.4064) (layer F.Cu) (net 10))
 (segment (start 147.64 123.16) (end 145.7 125.1) (width 0.762) (layer F.Cu) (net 10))
 (segment (start 147.64 120.87) (end 147.64 123.16) (width 0.762) (layer F.Cu) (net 10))
 (segment (start 145.7 125.1) (end 139.4 125.1) (width 0.762) (layer F.Cu) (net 10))
 (segment (start 138.525 125.975) (end 139.4 125.1) (width 0.762) (layer F.Cu) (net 10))
 (segment (start 137.2 125.975) (end 138.525 125.975) (width 0.762) (layer F.Cu) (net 10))
 (segment (start 143.145 111.495) (end 142.119238 111.495) (width 0.4) (layer F.Cu) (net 16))
 (segment (start 142.119238 111.495) (end 141.28 112.334238) (width 0.4) (layer F.Cu) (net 16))
 (segment (start 141.28 119.59) (end 142.56 120.87) (width 0.762) (layer F.Cu) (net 16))
 (segment (start 141.28 112.334238) (end 141.28 113.52) (width 0.4064) (layer F.Cu) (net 16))
 (segment (start 141.28 113.52) (end 141.28 119.59) (width 0.762) (layer F.Cu) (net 16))
 (segment (start 145.1 120.87) (end 143.145 118.915) (width 0.762) (layer F.Cu) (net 17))
 (segment (start 143.145 118.915) (end 143.145 112.445) (width 0.762) (layer F.Cu) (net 17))
 (segment (start 152.72 120.22) (end 152.72 120.87) (width 0.762) (layer F.Cu) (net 19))
 (segment (start 147.74 113.98) (end 147.74 115.24) (width 0.762) (layer F.Cu) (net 19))
 (segment (start 147.74 115.24) (end 152.72 120.22) (width 0.762) (layer F.Cu) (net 19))
 (segment (start 147.67 111.844238) (end 147.67 113.83) (width 0.4064) (layer F.Cu) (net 19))
 (segment (start 149.045 111.495) (end 148.019238 111.495) (width 0.4) (layer F.Cu) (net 19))
 (segment (start 148.019238 111.495) (end 147.67 111.844238) (width 0.4) (layer F.Cu) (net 19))
 (segment (start 149.045 110.845) (end 147.325 110.845) (width 0.4) (layer F.Cu) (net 18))
 (segment (start 147.325 110.845) (end 146.48 111.69) (width 0.4064) (layer F.Cu) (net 18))
 (segment (start 146.48 117.17) (end 150.18 120.87) (width 0.762) (layer F.Cu) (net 18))
 (segment (start 146.48 114) (end 146.48 117.17) (width 0.762) (layer F.Cu) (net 18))
 (segment (start 146.48 111.69) (end 146.48 114) (width 0.4064) (layer F.Cu) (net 18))
 (segment (start 123.2125 102.55) (end 123.2125 108.85) (width 0.4064) (layer F.Cu) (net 6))
 (segment (start 123.2125 101.85) (end 123.2125 102.55) (width 0.4064) (layer F.Cu) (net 6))
 (segment (start 130.057 108.458) (end 131.654 108.458) (width 0.762) (layer F.Cu) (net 7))
 (segment (start 130.057 107.933) (end 130.057 108.458) (width 0.762) (layer F.Cu) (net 7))
 (segment (start 131.44 104.07) (end 131.44 106.55) (width 0.762) (layer F.Cu) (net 7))
 (segment (start 131.44 106.55) (end 130.057 107.933) (width 0.762) (layer F.Cu) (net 7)))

